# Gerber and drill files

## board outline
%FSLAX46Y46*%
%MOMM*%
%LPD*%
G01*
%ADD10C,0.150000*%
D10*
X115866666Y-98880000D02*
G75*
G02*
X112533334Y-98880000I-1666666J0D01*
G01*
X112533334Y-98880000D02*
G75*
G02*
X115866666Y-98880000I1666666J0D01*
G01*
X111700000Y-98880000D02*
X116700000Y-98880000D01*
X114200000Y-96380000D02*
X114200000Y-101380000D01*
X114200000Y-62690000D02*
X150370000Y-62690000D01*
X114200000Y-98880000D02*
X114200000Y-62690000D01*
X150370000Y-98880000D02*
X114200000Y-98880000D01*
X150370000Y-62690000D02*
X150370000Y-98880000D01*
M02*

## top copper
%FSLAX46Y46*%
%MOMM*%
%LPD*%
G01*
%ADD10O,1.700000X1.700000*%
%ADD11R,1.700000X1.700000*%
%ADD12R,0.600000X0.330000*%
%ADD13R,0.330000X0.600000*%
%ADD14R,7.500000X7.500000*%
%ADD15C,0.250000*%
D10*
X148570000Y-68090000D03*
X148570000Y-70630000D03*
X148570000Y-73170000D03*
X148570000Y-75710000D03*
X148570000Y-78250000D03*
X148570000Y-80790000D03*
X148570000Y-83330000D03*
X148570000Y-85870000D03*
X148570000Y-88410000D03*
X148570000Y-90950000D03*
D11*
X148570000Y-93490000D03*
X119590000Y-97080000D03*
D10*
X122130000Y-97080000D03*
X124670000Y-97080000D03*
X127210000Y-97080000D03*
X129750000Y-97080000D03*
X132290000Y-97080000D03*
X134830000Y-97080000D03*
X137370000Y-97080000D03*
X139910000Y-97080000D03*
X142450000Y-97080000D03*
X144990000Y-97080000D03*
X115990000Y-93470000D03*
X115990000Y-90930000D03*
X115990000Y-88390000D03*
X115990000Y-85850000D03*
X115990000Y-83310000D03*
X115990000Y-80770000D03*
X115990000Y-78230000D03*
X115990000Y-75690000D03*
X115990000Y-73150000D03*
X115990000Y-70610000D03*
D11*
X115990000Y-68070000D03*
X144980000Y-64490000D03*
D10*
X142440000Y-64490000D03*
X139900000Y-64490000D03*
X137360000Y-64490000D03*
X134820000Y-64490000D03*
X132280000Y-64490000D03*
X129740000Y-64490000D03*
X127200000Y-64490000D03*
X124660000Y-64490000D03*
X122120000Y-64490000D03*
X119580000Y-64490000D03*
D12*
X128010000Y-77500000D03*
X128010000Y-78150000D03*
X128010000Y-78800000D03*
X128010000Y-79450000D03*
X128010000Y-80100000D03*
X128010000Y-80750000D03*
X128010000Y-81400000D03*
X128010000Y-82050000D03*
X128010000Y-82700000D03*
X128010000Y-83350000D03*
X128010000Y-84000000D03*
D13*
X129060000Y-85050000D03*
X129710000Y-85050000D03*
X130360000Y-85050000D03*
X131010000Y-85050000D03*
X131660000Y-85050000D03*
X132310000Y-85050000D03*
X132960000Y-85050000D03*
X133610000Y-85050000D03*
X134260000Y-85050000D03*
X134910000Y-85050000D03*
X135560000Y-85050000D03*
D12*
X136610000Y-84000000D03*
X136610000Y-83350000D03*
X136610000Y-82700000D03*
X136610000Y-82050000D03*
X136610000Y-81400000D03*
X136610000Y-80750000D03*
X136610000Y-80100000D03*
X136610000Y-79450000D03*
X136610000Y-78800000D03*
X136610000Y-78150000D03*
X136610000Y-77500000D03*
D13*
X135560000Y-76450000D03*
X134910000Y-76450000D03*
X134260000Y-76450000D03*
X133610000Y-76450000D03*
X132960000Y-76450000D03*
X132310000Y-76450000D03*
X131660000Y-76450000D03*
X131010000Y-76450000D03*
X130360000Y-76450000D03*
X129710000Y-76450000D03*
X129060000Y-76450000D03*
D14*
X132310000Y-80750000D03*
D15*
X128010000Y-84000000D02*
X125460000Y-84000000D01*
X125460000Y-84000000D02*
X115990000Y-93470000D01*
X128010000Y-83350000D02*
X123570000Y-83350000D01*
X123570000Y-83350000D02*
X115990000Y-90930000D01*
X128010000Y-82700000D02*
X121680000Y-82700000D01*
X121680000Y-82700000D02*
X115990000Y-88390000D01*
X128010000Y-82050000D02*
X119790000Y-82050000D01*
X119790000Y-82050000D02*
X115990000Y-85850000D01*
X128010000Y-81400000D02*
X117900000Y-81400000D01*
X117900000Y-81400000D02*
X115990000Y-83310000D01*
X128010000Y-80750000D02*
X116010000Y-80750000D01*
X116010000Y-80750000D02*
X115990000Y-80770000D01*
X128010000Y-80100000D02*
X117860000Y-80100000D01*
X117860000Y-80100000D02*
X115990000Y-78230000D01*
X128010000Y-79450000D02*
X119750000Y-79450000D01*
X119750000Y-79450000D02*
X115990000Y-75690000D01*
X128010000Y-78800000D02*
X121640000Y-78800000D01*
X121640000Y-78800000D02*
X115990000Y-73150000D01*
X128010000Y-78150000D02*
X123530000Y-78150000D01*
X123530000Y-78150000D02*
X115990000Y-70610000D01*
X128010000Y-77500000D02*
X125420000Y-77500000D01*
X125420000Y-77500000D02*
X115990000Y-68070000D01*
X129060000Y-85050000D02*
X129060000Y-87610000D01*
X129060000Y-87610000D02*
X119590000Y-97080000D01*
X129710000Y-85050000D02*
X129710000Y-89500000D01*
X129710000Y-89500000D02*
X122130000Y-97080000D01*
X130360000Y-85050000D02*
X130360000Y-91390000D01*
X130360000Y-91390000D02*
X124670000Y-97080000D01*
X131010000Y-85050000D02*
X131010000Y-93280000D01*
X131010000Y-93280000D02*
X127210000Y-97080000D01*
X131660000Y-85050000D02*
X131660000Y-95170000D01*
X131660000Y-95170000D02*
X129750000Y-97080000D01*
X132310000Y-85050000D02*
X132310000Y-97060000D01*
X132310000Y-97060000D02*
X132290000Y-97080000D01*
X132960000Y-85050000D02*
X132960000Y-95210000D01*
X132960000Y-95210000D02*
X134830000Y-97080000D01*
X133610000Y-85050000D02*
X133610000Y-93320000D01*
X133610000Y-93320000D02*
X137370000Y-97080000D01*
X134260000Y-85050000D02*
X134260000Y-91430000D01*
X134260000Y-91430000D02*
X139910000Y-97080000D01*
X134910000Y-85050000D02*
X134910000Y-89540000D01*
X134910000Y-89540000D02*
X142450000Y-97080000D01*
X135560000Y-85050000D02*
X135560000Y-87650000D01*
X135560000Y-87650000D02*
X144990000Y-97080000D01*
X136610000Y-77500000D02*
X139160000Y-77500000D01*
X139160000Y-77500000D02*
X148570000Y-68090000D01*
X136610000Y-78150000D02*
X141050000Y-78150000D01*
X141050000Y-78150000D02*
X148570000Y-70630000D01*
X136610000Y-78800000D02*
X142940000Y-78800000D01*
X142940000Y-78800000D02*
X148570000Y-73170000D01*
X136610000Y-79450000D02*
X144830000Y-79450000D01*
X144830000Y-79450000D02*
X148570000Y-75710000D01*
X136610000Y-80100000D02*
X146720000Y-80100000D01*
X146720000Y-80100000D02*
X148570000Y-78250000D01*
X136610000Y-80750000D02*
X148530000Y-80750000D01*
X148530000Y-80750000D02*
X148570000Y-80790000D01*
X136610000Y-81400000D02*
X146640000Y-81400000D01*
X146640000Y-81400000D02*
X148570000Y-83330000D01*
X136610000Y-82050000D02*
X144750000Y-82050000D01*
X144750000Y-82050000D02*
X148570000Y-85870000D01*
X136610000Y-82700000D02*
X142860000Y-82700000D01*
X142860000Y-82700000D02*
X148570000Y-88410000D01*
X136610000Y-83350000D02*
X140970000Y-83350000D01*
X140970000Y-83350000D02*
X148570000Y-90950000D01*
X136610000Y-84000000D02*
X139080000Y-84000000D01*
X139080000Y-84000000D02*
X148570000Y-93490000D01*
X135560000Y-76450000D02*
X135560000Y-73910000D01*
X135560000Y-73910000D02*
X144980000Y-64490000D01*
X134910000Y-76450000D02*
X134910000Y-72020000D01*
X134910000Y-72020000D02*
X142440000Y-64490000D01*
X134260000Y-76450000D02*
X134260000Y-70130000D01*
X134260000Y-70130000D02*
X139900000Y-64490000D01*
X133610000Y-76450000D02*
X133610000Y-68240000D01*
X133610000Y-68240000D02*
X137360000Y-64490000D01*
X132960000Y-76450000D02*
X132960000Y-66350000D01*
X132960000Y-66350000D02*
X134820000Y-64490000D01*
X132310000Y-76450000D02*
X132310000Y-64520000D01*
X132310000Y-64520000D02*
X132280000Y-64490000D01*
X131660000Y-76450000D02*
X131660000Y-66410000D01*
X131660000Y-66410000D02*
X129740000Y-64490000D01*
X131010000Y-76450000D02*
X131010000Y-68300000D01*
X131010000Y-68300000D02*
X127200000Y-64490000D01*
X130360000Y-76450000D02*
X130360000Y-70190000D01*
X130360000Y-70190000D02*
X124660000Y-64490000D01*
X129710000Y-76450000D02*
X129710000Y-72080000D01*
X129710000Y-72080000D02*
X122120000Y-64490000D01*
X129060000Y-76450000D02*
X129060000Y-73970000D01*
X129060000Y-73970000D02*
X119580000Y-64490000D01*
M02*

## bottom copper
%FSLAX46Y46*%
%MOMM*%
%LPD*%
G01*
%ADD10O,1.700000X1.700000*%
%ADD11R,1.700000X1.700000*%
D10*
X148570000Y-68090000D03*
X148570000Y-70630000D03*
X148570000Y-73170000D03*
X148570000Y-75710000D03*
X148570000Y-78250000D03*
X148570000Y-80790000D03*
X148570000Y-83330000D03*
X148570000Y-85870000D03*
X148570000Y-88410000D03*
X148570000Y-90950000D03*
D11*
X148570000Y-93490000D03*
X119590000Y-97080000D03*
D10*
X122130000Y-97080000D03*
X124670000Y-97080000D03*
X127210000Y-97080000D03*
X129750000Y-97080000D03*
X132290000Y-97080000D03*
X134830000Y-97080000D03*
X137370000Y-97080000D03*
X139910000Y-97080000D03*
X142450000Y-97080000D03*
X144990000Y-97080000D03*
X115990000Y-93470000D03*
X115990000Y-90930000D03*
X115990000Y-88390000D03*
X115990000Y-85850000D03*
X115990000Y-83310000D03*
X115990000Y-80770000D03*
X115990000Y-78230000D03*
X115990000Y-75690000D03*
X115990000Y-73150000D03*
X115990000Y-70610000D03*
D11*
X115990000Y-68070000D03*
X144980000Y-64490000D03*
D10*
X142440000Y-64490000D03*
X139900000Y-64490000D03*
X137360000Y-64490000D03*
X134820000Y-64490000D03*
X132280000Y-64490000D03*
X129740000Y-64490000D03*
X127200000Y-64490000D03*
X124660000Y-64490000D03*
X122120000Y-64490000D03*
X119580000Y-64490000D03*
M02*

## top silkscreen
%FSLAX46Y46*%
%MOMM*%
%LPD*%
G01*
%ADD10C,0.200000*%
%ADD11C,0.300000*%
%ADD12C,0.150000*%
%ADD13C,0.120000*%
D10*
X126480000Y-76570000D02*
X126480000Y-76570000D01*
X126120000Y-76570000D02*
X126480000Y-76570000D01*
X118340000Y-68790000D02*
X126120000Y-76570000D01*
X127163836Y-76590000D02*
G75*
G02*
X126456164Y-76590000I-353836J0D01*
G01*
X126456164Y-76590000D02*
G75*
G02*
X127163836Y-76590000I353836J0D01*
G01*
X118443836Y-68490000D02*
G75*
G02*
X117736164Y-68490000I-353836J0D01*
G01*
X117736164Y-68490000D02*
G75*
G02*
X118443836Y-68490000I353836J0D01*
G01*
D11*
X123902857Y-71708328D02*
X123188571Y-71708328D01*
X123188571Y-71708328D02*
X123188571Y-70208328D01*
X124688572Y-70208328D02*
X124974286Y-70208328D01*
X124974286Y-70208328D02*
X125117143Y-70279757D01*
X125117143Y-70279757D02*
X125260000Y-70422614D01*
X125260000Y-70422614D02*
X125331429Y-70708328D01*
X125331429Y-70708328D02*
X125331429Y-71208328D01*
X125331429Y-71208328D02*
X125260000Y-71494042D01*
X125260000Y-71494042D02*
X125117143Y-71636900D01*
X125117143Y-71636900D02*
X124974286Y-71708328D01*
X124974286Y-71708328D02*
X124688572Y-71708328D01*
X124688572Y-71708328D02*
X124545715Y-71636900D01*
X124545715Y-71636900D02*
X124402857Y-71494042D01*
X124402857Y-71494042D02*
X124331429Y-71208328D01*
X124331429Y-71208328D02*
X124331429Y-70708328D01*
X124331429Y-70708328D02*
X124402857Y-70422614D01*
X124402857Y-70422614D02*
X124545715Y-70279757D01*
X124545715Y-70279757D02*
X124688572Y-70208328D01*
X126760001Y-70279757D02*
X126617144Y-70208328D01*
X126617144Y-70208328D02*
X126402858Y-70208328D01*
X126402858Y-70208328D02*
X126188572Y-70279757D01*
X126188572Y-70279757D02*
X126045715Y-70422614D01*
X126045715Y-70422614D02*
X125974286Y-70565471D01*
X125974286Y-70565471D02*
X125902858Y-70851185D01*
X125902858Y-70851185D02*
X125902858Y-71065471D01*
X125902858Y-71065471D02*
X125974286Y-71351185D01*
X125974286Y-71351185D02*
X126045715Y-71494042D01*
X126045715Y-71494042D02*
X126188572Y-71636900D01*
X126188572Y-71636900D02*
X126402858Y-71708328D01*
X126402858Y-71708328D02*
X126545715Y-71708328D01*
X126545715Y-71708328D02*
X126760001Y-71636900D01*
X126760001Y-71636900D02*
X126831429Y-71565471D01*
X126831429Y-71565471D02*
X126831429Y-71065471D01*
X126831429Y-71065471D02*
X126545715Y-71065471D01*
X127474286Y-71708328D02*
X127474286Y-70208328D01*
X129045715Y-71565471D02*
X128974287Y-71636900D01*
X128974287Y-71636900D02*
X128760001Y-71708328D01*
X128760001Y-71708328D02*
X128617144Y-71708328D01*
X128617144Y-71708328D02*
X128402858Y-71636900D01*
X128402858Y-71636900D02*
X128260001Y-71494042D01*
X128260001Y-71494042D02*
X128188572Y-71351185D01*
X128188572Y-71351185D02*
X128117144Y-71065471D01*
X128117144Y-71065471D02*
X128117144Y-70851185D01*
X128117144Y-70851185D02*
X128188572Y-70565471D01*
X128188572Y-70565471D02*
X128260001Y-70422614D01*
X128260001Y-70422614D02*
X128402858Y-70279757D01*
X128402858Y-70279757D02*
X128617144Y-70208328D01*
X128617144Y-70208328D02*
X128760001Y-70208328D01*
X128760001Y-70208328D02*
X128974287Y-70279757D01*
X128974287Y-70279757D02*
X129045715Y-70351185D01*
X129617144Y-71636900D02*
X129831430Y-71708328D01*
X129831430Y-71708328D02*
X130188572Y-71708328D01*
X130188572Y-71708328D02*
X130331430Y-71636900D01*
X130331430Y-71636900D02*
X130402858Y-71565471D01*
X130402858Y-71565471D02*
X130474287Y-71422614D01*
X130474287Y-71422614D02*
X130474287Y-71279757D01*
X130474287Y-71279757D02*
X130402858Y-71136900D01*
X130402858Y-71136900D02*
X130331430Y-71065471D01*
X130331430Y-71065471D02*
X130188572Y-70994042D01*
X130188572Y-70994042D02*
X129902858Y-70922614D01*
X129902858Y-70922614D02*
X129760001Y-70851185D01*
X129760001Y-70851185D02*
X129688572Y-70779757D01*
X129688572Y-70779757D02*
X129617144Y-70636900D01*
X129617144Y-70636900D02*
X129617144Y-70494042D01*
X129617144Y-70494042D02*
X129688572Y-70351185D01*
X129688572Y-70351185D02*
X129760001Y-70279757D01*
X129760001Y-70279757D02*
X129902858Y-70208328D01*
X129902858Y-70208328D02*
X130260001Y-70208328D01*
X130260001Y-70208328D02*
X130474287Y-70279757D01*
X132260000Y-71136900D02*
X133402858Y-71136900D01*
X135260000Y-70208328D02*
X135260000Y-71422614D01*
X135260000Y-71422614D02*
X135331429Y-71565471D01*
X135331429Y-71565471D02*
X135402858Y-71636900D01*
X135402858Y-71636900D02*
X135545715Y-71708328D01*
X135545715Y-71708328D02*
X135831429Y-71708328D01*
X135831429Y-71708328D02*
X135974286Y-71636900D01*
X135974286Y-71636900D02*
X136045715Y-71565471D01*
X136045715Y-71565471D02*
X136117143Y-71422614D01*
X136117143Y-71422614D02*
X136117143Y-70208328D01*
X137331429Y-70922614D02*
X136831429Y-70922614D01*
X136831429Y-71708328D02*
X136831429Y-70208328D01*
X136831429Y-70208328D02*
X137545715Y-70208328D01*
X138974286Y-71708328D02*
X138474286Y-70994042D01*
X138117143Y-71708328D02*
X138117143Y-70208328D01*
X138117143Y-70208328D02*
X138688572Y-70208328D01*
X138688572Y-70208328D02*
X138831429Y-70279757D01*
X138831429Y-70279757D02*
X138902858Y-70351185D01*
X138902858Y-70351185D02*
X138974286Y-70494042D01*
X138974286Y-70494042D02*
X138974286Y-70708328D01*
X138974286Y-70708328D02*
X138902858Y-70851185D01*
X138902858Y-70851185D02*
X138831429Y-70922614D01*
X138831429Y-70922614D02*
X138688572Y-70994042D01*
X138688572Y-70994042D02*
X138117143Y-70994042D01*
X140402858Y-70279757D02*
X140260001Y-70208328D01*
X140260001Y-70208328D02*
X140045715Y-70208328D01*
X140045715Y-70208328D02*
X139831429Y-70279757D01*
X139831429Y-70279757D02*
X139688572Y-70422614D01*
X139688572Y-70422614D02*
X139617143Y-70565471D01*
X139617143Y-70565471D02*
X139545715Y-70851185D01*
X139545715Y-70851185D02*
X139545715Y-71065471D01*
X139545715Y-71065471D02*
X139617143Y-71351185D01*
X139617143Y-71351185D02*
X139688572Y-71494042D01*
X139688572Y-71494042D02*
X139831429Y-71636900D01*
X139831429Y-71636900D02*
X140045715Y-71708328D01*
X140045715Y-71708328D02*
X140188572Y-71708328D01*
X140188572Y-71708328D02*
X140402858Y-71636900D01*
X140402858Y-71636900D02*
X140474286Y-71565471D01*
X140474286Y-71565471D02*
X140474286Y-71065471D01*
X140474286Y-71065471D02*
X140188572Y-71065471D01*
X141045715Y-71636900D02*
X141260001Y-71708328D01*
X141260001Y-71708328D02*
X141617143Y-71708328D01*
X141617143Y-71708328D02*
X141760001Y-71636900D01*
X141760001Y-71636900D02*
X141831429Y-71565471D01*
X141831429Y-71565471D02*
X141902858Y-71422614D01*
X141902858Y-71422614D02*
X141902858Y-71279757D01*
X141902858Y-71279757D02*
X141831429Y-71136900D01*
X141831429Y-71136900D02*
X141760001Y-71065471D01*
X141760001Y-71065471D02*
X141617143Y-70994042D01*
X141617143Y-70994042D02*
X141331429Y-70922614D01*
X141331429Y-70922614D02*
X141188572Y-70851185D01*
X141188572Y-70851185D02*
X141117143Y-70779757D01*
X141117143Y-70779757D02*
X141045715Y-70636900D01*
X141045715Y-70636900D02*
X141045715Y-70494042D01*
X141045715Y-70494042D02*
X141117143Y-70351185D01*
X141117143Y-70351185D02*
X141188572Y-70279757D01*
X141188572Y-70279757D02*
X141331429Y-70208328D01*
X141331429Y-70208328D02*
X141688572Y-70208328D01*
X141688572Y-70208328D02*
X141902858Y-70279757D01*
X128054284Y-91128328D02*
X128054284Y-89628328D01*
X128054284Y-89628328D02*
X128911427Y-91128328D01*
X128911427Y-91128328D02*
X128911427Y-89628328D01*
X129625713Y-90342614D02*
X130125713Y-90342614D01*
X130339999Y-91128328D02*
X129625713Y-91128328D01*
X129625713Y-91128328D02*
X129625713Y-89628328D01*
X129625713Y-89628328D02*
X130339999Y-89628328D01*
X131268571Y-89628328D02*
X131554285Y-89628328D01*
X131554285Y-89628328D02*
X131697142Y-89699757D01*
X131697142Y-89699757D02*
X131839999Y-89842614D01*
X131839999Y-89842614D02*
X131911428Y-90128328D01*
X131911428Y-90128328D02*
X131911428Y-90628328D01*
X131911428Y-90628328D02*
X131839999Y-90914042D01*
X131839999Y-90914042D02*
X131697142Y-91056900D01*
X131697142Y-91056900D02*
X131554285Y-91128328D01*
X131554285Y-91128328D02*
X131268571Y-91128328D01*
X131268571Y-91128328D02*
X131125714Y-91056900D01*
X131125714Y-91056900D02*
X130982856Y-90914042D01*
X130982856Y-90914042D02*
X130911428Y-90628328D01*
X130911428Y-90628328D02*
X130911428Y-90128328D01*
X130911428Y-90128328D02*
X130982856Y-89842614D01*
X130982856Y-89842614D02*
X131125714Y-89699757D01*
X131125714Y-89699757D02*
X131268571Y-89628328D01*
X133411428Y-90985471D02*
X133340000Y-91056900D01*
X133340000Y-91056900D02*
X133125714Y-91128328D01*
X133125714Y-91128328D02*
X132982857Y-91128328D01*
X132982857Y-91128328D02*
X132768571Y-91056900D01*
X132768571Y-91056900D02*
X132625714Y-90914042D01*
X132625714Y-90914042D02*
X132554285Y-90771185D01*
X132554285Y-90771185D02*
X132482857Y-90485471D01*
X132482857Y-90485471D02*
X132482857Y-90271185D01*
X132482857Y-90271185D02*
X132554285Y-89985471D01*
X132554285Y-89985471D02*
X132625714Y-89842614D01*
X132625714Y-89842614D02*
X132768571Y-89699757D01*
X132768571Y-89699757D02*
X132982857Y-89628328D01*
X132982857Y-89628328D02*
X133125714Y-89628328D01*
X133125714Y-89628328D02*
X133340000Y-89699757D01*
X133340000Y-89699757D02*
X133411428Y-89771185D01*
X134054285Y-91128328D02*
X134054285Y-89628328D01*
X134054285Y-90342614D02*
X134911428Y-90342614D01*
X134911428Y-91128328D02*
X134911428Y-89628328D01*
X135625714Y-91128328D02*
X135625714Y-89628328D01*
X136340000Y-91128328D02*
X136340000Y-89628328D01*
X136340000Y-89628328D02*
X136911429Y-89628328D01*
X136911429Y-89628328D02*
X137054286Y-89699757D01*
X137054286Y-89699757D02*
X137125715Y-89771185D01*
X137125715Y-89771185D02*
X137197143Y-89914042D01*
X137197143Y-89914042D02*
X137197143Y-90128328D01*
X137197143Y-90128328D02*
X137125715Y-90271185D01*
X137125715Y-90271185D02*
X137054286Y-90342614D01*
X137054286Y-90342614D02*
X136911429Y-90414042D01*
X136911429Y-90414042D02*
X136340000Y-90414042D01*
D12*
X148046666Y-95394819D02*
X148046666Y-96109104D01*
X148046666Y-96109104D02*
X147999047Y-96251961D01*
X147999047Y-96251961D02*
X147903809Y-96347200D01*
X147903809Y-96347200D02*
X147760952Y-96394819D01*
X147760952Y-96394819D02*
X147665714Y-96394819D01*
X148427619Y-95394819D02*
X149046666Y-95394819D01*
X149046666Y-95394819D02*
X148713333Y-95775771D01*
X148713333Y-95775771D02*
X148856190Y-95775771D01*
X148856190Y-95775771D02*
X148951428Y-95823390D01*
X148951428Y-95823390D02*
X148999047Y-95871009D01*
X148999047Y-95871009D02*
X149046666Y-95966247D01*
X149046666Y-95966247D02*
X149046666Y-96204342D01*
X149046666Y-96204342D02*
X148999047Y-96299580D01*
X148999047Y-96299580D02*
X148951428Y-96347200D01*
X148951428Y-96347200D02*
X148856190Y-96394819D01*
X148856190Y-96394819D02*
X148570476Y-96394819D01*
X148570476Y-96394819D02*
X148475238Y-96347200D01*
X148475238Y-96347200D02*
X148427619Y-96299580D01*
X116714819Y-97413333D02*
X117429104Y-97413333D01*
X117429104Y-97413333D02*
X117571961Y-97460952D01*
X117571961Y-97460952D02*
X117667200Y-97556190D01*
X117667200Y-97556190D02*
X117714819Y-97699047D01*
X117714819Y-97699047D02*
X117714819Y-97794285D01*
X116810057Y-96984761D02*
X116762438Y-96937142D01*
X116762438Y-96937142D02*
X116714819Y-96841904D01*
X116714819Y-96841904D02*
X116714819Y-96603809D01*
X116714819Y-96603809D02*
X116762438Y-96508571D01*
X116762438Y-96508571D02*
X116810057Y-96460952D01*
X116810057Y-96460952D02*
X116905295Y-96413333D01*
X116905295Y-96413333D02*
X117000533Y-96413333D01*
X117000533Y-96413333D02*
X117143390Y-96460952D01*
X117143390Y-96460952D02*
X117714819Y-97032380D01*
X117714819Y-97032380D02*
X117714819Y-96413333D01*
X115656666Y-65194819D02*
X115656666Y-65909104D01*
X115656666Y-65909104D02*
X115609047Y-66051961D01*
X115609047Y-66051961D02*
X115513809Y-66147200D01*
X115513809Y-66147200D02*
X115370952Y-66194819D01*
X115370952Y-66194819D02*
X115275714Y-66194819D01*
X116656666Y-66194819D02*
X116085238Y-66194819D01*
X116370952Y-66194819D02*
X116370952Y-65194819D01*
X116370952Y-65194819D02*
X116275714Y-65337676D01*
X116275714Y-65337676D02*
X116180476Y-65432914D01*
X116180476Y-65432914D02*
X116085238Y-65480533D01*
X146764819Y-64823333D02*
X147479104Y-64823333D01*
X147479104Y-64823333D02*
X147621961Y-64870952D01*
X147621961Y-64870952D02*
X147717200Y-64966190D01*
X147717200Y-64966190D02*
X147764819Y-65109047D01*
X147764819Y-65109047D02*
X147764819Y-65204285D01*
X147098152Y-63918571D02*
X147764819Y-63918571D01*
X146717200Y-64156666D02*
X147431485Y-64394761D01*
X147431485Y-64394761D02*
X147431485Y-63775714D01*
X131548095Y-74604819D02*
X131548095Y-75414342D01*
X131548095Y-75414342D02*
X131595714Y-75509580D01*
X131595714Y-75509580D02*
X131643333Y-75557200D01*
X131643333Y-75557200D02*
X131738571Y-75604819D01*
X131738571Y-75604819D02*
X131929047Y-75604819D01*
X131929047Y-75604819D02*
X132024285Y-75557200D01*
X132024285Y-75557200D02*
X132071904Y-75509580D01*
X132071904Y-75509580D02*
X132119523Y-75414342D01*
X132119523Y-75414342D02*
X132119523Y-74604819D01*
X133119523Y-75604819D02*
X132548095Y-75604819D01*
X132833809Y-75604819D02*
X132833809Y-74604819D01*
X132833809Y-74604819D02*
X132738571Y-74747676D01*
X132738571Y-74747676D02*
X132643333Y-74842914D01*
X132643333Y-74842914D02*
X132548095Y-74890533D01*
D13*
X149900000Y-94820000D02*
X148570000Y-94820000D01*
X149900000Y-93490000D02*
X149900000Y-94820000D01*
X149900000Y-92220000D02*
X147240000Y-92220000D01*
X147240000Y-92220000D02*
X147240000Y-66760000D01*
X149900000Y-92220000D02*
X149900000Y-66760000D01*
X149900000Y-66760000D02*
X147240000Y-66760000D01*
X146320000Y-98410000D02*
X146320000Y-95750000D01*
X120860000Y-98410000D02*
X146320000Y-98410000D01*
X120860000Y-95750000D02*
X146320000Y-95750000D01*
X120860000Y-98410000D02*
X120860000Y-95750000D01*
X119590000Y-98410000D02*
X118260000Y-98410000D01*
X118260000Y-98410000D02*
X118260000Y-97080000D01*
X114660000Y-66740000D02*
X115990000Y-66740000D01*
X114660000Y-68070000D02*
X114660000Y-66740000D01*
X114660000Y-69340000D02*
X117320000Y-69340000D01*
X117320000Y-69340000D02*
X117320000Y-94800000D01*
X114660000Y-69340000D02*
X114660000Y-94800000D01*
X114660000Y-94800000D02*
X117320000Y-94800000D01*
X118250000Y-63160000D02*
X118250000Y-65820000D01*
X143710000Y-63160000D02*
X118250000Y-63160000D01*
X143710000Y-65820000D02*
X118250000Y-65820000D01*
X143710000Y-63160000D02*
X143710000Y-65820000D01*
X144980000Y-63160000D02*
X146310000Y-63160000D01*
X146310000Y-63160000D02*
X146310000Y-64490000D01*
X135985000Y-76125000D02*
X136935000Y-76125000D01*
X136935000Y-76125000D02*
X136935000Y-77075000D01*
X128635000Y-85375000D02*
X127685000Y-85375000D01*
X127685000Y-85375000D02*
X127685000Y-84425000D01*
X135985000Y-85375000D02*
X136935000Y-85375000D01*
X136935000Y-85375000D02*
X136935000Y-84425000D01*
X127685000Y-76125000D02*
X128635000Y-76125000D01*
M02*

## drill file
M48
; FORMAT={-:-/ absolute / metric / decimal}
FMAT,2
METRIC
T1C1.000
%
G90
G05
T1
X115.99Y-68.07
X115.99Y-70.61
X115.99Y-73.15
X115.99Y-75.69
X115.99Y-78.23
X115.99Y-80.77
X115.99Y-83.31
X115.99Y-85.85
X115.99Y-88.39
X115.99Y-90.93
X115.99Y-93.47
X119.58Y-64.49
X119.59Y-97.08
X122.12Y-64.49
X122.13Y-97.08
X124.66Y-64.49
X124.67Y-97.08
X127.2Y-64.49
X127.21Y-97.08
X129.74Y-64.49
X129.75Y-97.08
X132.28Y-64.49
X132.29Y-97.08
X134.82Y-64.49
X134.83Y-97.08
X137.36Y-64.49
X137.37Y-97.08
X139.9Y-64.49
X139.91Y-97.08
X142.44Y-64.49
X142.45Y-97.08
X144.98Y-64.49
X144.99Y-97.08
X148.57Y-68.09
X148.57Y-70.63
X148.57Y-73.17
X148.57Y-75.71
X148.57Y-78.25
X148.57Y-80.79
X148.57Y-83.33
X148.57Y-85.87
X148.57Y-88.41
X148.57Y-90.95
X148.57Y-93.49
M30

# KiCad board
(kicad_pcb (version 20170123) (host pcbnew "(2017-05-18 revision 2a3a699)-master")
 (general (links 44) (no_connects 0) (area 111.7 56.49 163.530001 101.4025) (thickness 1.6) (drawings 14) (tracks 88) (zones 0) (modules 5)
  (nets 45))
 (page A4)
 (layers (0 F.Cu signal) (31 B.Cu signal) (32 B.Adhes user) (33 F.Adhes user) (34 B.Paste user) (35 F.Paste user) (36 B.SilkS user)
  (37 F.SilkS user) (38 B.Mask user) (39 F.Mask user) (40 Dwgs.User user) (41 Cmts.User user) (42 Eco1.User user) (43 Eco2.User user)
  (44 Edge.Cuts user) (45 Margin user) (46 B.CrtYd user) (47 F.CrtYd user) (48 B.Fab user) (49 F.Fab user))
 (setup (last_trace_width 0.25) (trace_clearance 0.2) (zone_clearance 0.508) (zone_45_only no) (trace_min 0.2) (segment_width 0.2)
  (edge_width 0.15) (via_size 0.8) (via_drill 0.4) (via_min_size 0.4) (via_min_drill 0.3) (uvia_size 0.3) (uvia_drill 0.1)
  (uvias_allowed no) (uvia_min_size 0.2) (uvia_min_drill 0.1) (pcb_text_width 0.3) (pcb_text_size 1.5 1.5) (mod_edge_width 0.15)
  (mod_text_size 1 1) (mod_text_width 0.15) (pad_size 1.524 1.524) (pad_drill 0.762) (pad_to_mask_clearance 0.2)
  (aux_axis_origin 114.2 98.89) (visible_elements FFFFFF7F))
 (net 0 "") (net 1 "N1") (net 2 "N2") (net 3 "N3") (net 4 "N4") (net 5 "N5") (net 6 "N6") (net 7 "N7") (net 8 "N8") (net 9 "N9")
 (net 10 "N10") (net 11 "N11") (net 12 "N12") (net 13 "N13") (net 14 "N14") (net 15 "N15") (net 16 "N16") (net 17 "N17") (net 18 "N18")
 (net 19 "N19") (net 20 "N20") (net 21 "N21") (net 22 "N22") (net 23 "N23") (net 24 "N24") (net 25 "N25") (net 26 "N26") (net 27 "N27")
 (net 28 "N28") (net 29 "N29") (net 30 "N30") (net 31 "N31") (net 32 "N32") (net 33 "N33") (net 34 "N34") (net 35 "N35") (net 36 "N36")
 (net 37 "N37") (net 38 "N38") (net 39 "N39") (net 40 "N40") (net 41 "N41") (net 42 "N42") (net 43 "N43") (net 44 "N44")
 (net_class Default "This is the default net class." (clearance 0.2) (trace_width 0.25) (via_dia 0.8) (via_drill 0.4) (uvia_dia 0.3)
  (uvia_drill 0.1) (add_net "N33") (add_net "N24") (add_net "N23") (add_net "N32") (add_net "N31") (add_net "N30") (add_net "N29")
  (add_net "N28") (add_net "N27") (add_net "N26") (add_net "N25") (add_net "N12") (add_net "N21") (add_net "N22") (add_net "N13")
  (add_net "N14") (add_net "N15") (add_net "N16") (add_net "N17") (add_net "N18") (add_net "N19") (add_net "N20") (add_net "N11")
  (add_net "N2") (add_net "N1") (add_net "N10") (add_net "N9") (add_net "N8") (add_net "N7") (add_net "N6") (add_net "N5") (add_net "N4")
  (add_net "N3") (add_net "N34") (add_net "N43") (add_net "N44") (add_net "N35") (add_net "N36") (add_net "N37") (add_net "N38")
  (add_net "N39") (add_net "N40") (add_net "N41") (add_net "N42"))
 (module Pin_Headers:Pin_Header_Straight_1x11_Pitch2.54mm (layer F.Cu) (at 148.57 93.49 180)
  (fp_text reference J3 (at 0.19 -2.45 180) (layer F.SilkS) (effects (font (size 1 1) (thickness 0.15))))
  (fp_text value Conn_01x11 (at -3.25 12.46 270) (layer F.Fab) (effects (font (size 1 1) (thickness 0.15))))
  (fp_line (start -1.33 -1.33) (end 0 -1.33) (layer F.SilkS) (width 0.12))
  (fp_line (start -1.33 0) (end -1.33 -1.33) (layer F.SilkS) (width 0.12))
  (fp_line (start -1.33 1.27) (end 1.33 1.27) (layer F.SilkS) (width 0.12))
  (fp_line (start 1.33 1.27) (end 1.33 26.73) (layer F.SilkS) (width 0.12))
  (fp_line (start -1.33 1.27) (end -1.33 26.73) (layer F.SilkS) (width 0.12))
  (fp_line (start -1.33 26.73) (end 1.33 26.73) (layer F.SilkS) (width 0.12))
  (pad 11 thru_hole oval (at 0 25.4 180) (size 1.7 1.7) (drill 1) (layers *.Cu *.Mask) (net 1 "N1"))
  (pad 10 thru_hole oval (at 0 22.86 180) (size 1.7 1.7) (drill 1) (layers *.Cu *.Mask) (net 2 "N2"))
  (pad 9 thru_hole oval (at 0 20.32 180) (size 1.7 1.7) (drill 1) (layers *.Cu *.Mask) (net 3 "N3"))
  (pad 8 thru_hole oval (at 0 17.78 180) (size 1.7 1.7) (drill 1) (layers *.Cu *.Mask) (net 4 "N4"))
  (pad 7 thru_hole oval (at 0 15.24 180) (size 1.7 1.7) (drill 1) (layers *.Cu *.Mask) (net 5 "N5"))
  (pad 6 thru_hole oval (at 0 12.7 180) (size 1.7 1.7) (drill 1) (layers *.Cu *.Mask) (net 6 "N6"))
  (pad 5 thru_hole oval (at 0 10.16 180) (size 1.7 1.7) (drill 1) (layers *.Cu *.Mask) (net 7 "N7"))
  (pad 4 thru_hole oval (at 0 7.62 180) (size 1.7 1.7) (drill 1) (layers *.Cu *.Mask) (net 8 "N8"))
  (pad 3 thru_hole oval (at 0 5.08 180) (size 1.7 1.7) (drill 1) (layers *.Cu *.Mask) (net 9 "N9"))
  (pad 2 thru_hole oval (at 0 2.54 180) (size 1.7 1.7) (drill 1) (layers *.Cu *.Mask) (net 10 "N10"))
  (pad 1 thru_hole rect (at 0 0 180) (size 1.7 1.7) (drill 1) (layers *.Cu *.Mask) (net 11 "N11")))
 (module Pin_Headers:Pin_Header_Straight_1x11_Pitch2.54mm (layer F.Cu) (at 119.59 97.08 90)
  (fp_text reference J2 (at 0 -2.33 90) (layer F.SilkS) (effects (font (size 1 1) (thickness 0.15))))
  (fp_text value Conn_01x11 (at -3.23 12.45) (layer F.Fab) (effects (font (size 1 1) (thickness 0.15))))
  (fp_line (start -1.33 26.73) (end 1.33 26.73) (layer F.SilkS) (width 0.12))
  (fp_line (start -1.33 1.27) (end -1.33 26.73) (layer F.SilkS) (width 0.12))
  (fp_line (start 1.33 1.27) (end 1.33 26.73) (layer F.SilkS) (width 0.12))
  (fp_line (start -1.33 1.27) (end 1.33 1.27) (layer F.SilkS) (width 0.12))
  (fp_line (start -1.33 0) (end -1.33 -1.33) (layer F.SilkS) (width 0.12))
  (fp_line (start -1.33 -1.33) (end 0 -1.33) (layer F.SilkS) (width 0.12))
  (pad 1 thru_hole rect (at 0 0 90) (size 1.7 1.7) (drill 1) (layers *.Cu *.Mask) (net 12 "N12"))
  (pad 2 thru_hole oval (at 0 2.54 90) (size 1.7 1.7) (drill 1) (layers *.Cu *.Mask) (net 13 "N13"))
  (pad 3 thru_hole oval (at 0 5.08 90) (size 1.7 1.7) (drill 1) (layers *.Cu *.Mask) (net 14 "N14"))
  (pad 4 thru_hole oval (at 0 7.62 90) (size 1.7 1.7) (drill 1) (layers *.Cu *.Mask) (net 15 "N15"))
  (pad 5 thru_hole oval (at 0 10.16 90) (size 1.7 1.7) (drill 1) (layers *.Cu *.Mask) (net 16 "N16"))
  (pad 6 thru_hole oval (at 0 12.7 90) (size 1.7 1.7) (drill 1) (layers *.Cu *.Mask) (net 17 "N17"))
  (pad 7 thru_hole oval (at 0 15.24 90) (size 1.7 1.7) (drill 1) (layers *.Cu *.Mask) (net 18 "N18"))
  (pad 8 thru_hole oval (at 0 17.78 90) (size 1.7 1.7) (drill 1) (layers *.Cu *.Mask) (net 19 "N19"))
  (pad 9 thru_hole oval (at 0 20.32 90) (size 1.7 1.7) (drill 1) (layers *.Cu *.Mask) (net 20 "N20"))
  (pad 10 thru_hole oval (at 0 22.86 90) (size 1.7 1.7) (drill 1) (layers *.Cu *.Mask) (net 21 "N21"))
  (pad 11 thru_hole oval (at 0 25.4 90) (size 1.7 1.7) (drill 1) (layers *.Cu *.Mask) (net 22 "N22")))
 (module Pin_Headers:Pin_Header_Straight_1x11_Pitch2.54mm (layer F.Cu) (at 115.99 68.07)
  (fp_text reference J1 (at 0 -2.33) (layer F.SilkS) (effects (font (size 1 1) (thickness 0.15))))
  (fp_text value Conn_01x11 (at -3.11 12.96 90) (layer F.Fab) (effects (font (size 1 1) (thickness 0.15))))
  (fp_line (start -1.33 -1.33) (end 0 -1.33) (layer F.SilkS) (width 0.12))
  (fp_line (start -1.33 0) (end -1.33 -1.33) (layer F.SilkS) (width 0.12))
  (fp_line (start -1.33 1.27) (end 1.33 1.27) (layer F.SilkS) (width 0.12))
  (fp_line (start 1.33 1.27) (end 1.33 26.73) (layer F.SilkS) (width 0.12))
  (fp_line (start -1.33 1.27) (end -1.33 26.73) (layer F.SilkS) (width 0.12))
  (fp_line (start -1.33 26.73) (end 1.33 26.73) (layer F.SilkS) (width 0.12))
  (pad 11 thru_hole oval (at 0 25.4) (size 1.7 1.7) (drill 1) (layers *.Cu *.Mask) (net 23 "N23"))
  (pad 10 thru_hole oval (at 0 22.86) (size 1.7 1.7) (drill 1) (layers *.Cu *.Mask) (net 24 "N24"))
  (pad 9 thru_hole oval (at 0 20.32) (size 1.7 1.7) (drill 1) (layers *.Cu *.Mask) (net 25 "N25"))
  (pad 8 thru_hole oval (at 0 17.78) (size 1.7 1.7) (drill 1) (layers *.Cu *.Mask) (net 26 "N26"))
  (pad 7 thru_hole oval (at 0 15.24) (size 1.7 1.7) (drill 1) (layers *.Cu *.Mask) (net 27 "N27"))
  (pad 6 thru_hole oval (at 0 12.7) (size 1.7 1.7) (drill 1) (layers *.Cu *.Mask) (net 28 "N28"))
  (pad 5 thru_hole oval (at 0 10.16) (size 1.7 1.7) (drill 1) (layers *.Cu *.Mask) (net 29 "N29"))
  (pad 4 thru_hole oval (at 0 7.62) (size 1.7 1.7) (drill 1) (layers *.Cu *.Mask) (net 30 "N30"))
  (pad 3 thru_hole oval (at 0 5.08) (size 1.7 1.7) (drill 1) (layers *.Cu *.Mask) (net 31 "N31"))
  (pad 2 thru_hole oval (at 0 2.54) (size 1.7 1.7) (drill 1) (layers *.Cu *.Mask) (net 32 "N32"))
  (pad 1 thru_hole rect (at 0 0) (size 1.7 1.7) (drill 1) (layers *.Cu *.Mask) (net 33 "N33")))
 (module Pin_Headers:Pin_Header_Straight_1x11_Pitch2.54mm (layer F.Cu) (at 144.98 64.49 270)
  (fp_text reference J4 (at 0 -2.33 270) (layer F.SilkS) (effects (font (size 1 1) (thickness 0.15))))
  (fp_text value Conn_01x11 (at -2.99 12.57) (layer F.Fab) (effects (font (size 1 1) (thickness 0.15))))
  (fp_line (start -1.33 26.73) (end 1.33 26.73) (layer F.SilkS) (width 0.12))
  (fp_line (start -1.33 1.27) (end -1.33 26.73) (layer F.SilkS) (width 0.12))
  (fp_line (start 1.33 1.27) (end 1.33 26.73) (layer F.SilkS) (width 0.12))
  (fp_line (start -1.33 1.27) (end 1.33 1.27) (layer F.SilkS) (width 0.12))
  (fp_line (start -1.33 0) (end -1.33 -1.33) (layer F.SilkS) (width 0.12))
  (fp_line (start -1.33 -1.33) (end 0 -1.33) (layer F.SilkS) (width 0.12))
  (pad 1 thru_hole rect (at 0 0 270) (size 1.7 1.7) (drill 1) (layers *.Cu *.Mask) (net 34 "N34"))
  (pad 2 thru_hole oval (at 0 2.54 270) (size 1.7 1.7) (drill 1) (layers *.Cu *.Mask) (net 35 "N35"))
  (pad 3 thru_hole oval (at 0 5.08 270) (size 1.7 1.7) (drill 1) (layers *.Cu *.Mask) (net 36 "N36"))
  (pad 4 thru_hole oval (at 0 7.62 270) (size 1.7 1.7) (drill 1) (layers *.Cu *.Mask) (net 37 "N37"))
  (pad 5 thru_hole oval (at 0 10.16 270) (size 1.7 1.7) (drill 1) (layers *.Cu *.Mask) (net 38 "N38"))
  (pad 6 thru_hole oval (at 0 12.7 270) (size 1.7 1.7) (drill 1) (layers *.Cu *.Mask) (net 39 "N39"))
  (pad 7 thru_hole oval (at 0 15.24 270) (size 1.7 1.7) (drill 1) (layers *.Cu *.Mask) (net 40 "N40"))
  (pad 8 thru_hole oval (at 0 17.78 270) (size 1.7 1.7) (drill 1) (layers *.Cu *.Mask) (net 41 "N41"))
  (pad 9 thru_hole oval (at 0 20.32 270) (size 1.7 1.7) (drill 1) (layers *.Cu *.Mask) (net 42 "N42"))
  (pad 10 thru_hole oval (at 0 22.86 270) (size 1.7 1.7) (drill 1) (layers *.Cu *.Mask) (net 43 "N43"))
  (pad 11 thru_hole oval (at 0 25.4 270) (size 1.7 1.7) (drill 1) (layers *.Cu *.Mask) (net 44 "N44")))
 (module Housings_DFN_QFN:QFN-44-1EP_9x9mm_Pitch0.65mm (layer F.Cu) (at 132.31 80.75)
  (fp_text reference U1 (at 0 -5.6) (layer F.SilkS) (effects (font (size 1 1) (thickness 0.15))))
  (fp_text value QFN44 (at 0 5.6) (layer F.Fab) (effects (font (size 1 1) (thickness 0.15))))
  (fp_line (start 3.675 -4.625) (end 4.625 -4.625) (layer F.SilkS) (width 0.12))
  (fp_line (start 4.625 -4.625) (end 4.625 -3.675) (layer F.SilkS) (width 0.12))
  (fp_line (start -3.675 4.625) (end -4.625 4.625) (layer F.SilkS) (width 0.12))
  (fp_line (start -4.625 4.625) (end -4.625 3.675) (layer F.SilkS) (width 0.12))
  (fp_line (start 3.675 4.625) (end 4.625 4.625) (layer F.SilkS) (width 0.12))
  (fp_line (start 4.625 4.625) (end 4.625 3.675) (layer F.SilkS) (width 0.12))
  (fp_line (start -4.625 -4.625) (end -3.675 -4.625) (layer F.SilkS) (width 0.12))
  (pad 1 smd rect (at -4.3 -3.25) (size 0.6 0.33) (layers F.Cu F.Paste F.Mask) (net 33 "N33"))
  (pad 2 smd rect (at -4.3 -2.6) (size 0.6 0.33) (layers F.Cu F.Paste F.Mask) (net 32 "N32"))
  (pad 3 smd rect (at -4.3 -1.95) (size 0.6 0.33) (layers F.Cu F.Paste F.Mask) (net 31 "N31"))
  (pad 4 smd rect (at -4.3 -1.3) (size 0.6 0.33) (layers F.Cu F.Paste F.Mask) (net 30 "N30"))
  (pad 5 smd rect (at -4.3 -0.65) (size 0.6 0.33) (layers F.Cu F.Paste F.Mask) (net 29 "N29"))
  (pad 6 smd rect (at -4.3 0) (size 0.6 0.33) (layers F.Cu F.Paste F.Mask) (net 28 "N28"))
  (pad 7 smd rect (at -4.3 0.65) (size 0.6 0.33) (layers F.Cu F.Paste F.Mask) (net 27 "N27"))
  (pad 8 smd rect (at -4.3 1.3) (size 0.6 0.33) (layers F.Cu F.Paste F.Mask) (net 26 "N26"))
  (pad 9 smd rect (at -4.3 1.95) (size 0.6 0.33) (layers F.Cu F.Paste F.Mask) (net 25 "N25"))
  (pad 10 smd rect (at -4.3 2.6) (size 0.6 0.33) (layers F.Cu F.Paste F.Mask) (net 24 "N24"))
  (pad 11 smd rect (at -4.3 3.25) (size 0.6 0.33) (layers F.Cu F.Paste F.Mask) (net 23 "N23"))
  (pad 12 smd rect (at -3.25 4.3 90) (size 0.6 0.33) (layers F.Cu F.Paste F.Mask) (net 12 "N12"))
  (pad 13 smd rect (at -2.6 4.3 90) (size 0.6 0.33) (layers F.Cu F.Paste F.Mask) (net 13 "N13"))
  (pad 14 smd rect (at -1.95 4.3 90) (size 0.6 0.33) (layers F.Cu F.Paste F.Mask) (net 14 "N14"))
  (pad 15 smd rect (at -1.3 4.3 90) (size 0.6 0.33) (layers F.Cu F.Paste F.Mask) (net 15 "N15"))
  (pad 16 smd rect (at -0.65 4.3 90) (size 0.6 0.33) (layers F.Cu F.Paste F.Mask) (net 16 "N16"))
  (pad 17 smd rect (at 0 4.3 90) (size 0.6 0.33) (layers F.Cu F.Paste F.Mask) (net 17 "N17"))
  (pad 18 smd rect (at 0.65 4.3 90) (size 0.6 0.33) (layers F.Cu F.Paste F.Mask) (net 18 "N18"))
  (pad 19 smd rect (at 1.3 4.3 90) (size 0.6 0.33) (layers F.Cu F.Paste F.Mask) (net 19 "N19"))
  (pad 20 smd rect (at 1.95 4.3 90) (size 0.6 0.33) (layers F.Cu F.Paste F.Mask) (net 20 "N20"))
  (pad 21 smd rect (at 2.6 4.3 90) (size 0.6 0.33) (layers F.Cu F.Paste F.Mask) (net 21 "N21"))
  (pad 22 smd rect (at 3.25 4.3 90) (size 0.6 0.33) (layers F.Cu F.Paste F.Mask) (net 22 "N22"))
  (pad 23 smd rect (at 4.3 3.25) (size 0.6 0.33) (layers F.Cu F.Paste F.Mask) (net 11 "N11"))
  (pad 24 smd rect (at 4.3 2.6) (size 0.6 0.33) (layers F.Cu F.Paste F.Mask) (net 10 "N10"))
  (pad 25 smd rect (at 4.3 1.95) (size 0.6 0.33) (layers F.Cu F.Paste F.Mask) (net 9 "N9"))
  (pad 26 smd rect (at 4.3 1.3) (size 0.6 0.33) (layers F.Cu F.Paste F.Mask) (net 8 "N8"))
  (pad 27 smd rect (at 4.3 0.65) (size 0.6 0.33) (layers F.Cu F.Paste F.Mask) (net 7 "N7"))
  (pad 28 smd rect (at 4.3 0) (size 0.6 0.33) (layers F.Cu F.Paste F.Mask) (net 6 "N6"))
  (pad 29 smd rect (at 4.3 -0.65) (size 0.6 0.33) (layers F.Cu F.Paste F.Mask) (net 5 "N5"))
  (pad 30 smd rect (at 4.3 -1.3) (size 0.6 0.33) (layers F.Cu F.Paste F.Mask) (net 4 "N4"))
  (pad 31 smd rect (at 4.3 -1.95) (size 0.6 0.33) (layers F.Cu F.Paste F.Mask) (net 3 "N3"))
  (pad 32 smd rect (at 4.3 -2.6) (size 0.6 0.33) (layers F.Cu F.Paste F.Mask) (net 2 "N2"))
  (pad 33 smd rect (at 4.3 -3.25) (size 0.6 0.33) (layers F.Cu F.Paste F.Mask) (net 1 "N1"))
  (pad 34 smd rect (at 3.25 -4.3 90) (size 0.6 0.33) (layers F.Cu F.Paste F.Mask) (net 34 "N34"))
  (pad 35 smd rect (at 2.6 -4.3 90) (size 0.6 0.33) (layers F.Cu F.Paste F.Mask) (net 35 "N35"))
  (pad 36 smd rect (at 1.95 -4.3 90) (size 0.6 0.33) (layers F.Cu F.Paste F.Mask) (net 36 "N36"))
  (pad 37 smd rect (at 1.3 -4.3 90) (size 0.6 0.33) (layers F.Cu F.Paste F.Mask) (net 37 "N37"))
  (pad 38 smd rect (at 0.65 -4.3 90) (size 0.6 0.33) (layers F.Cu F.Paste F.Mask) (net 38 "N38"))
  (pad 39 smd rect (at 0 -4.3 90) (size 0.6 0.33) (layers F.Cu F.Paste F.Mask) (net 39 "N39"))
  (pad 40 smd rect (at -0.65 -4.3 90) (size 0.6 0.33) (layers F.Cu F.Paste F.Mask) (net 40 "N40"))
  (pad 41 smd rect (at -1.3 -4.3 90) (size 0.6 0.33) (layers F.Cu F.Paste F.Mask) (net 41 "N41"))
  (pad 42 smd rect (at -1.95 -4.3 90) (size 0.6 0.33) (layers F.Cu F.Paste F.Mask) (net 42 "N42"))
  (pad 43 smd rect (at -2.6 -4.3 90) (size 0.6 0.33) (layers F.Cu F.Paste F.Mask) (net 43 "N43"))
  (pad 44 smd rect (at -3.25 -4.3 90) (size 0.6 0.33) (layers F.Cu F.Paste F.Mask) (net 44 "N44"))
  (pad 45 smd rect (at 0 0) (size 7.5 7.5) (layers F.Cu F.Mask))
  (pad "" smd rect (at -1.875 -1.875) (size 2.65 2.65) (layers F.Paste))
  (pad "" smd rect (at -1.875 1.875) (size 2.65 2.65) (layers F.Paste))
  (pad "" smd rect (at 1.875 -1.875) (size 2.65 2.65) (layers F.Paste))
  (pad "" smd rect (at 1.875 1.875) (size 2.65 2.65) (layers F.Paste)))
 (gr_line (start 126.48 76.57) (end 126.48 76.57) (layer F.SilkS) (width 0.2))
 (gr_line (start 126.12 76.57) (end 126.48 76.57) (layer F.SilkS) (width 0.2))
 (gr_line (start 118.34 68.79) (end 126.12 76.57) (layer F.SilkS) (width 0.2))
 (gr_circle (center 126.81 76.59) (end 126.55 76.35) (layer F.SilkS) (width 0.2))
 (gr_circle (center 118.09 68.49) (end 117.83 68.25) (layer F.SilkS) (width 0.2))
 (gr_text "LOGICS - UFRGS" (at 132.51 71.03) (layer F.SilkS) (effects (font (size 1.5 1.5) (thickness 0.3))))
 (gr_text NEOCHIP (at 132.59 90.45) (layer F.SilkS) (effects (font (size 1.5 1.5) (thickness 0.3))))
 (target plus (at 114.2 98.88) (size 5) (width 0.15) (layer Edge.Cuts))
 (gr_line (start 114.2 62.69) (end 150.37 62.69) (layer Edge.Cuts) (width 0.15))
 (gr_line (start 114.2 98.88) (end 114.2 62.69) (layer Edge.Cuts) (width 0.15))
 (gr_line (start 150.37 98.88) (end 114.2 98.88) (layer Edge.Cuts) (width 0.15))
 (gr_line (start 150.37 62.69) (end 150.37 98.88) (layer Edge.Cuts) (width 0.15))
 (segment (start 128.01 84) (end 125.46 84) (width 0.25) (layer F.Cu) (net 23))
 (segment (start 125.46 84) (end 115.99 93.47) (width 0.25) (layer F.Cu) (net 23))
 (segment (start 128.01 83.35) (end 123.57 83.35) (width 0.25) (layer F.Cu) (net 24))
 (segment (start 123.57 83.35) (end 115.99 90.93) (width 0.25) (layer F.Cu) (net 24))
 (segment (start 128.01 82.7) (end 121.68 82.7) (width 0.25) (layer F.Cu) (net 25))
 (segment (start 121.68 82.7) (end 115.99 88.39) (width 0.25) (layer F.Cu) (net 25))
 (segment (start 128.01 82.05) (end 119.79 82.05) (width 0.25) (layer F.Cu) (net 26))
 (segment (start 119.79 82.05) (end 115.99 85.85) (width 0.25) (layer F.Cu) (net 26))
 (segment (start 128.01 81.4) (end 117.9 81.4) (width 0.25) (layer F.Cu) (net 27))
 (segment (start 117.9 81.4) (end 115.99 83.31) (width 0.25) (layer F.Cu) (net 27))
 (segment (start 128.01 80.75) (end 116.01 80.75) (width 0.25) (layer F.Cu) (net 28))
 (segment (start 116.01 80.75) (end 115.99 80.77) (width 0.25) (layer F.Cu) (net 28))
 (segment (start 128.01 80.1) (end 117.86 80.1) (width 0.25) (layer F.Cu) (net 29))
 (segment (start 117.86 80.1) (end 115.99 78.23) (width 0.25) (layer F.Cu) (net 29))
 (segment (start 128.01 79.45) (end 119.75 79.45) (width 0.25) (layer F.Cu) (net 30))
 (segment (start 119.75 79.45) (end 115.99 75.69) (width 0.25) (layer F.Cu) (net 30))
 (segment (start 128.01 78.8) (end 121.64 78.8) (width 0.25) (layer F.Cu) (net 31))
 (segment (start 121.64 78.8) (end 115.99 73.15) (width 0.25) (layer F.Cu) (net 31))
 (segment (start 128.01 78.15) (end 123.53 78.15) (width 0.25) (layer F.Cu) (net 32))
 (segment (start 123.53 78.15) (end 115.99 70.61) (width 0.25) (layer F.Cu) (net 32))
 (segment (start 128.01 77.5) (end 125.42 77.5) (width 0.25) (layer F.Cu) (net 33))
 (segment (start 125.42 77.5) (end 115.99 68.07) (width 0.25) (layer F.Cu) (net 33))
 (segment (start 129.06 85.05) (end 129.06 87.61) (width 0.25) (layer F.Cu) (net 12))
 (segment (start 129.06 87.61) (end 119.59 97.08) (width 0.25) (layer F.Cu) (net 12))
 (segment (start 129.71 85.05) (end 129.71 89.5) (width 0.25) (layer F.Cu) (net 13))
 (segment (start 129.71 89.5) (end 122.13 97.08) (width 0.25) (layer F.Cu) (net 13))
 (segment (start 130.36 85.05) (end 130.36 91.39) (width 0.25) (layer F.Cu) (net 14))
 (segment (start 130.36 91.39) (end 124.67 97.08) (width 0.25) (layer F.Cu) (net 14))
 (segment (start 131.01 85.05) (end 131.01 93.28) (width 0.25) (layer F.Cu) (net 15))
 (segment (start 131.01 93.28) (end 127.21 97.08) (width 0.25) (layer F.Cu) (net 15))
 (segment (start 131.66 85.05) (end 131.66 95.17) (width 0.25) (layer F.Cu) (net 16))
 (segment (start 131.66 95.17) (end 129.75 97.08) (width 0.25) (layer F.Cu) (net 16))
 (segment (start 132.31 85.05) (end 132.31 97.06) (width 0.25) (layer F.Cu) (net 17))
 (segment (start 132.31 97.06) (end 132.29 97.08) (width 0.25) (layer F.Cu) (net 17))
 (segment (start 132.96 85.05) (end 132.96 95.21) (width 0.25) (layer F.Cu) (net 18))
 (segment (start 132.96 95.21) (end 134.83 97.08) (width 0.25) (layer F.Cu) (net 18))
 (segment (start 133.61 85.05) (end 133.61 93.32) (width 0.25) (layer F.Cu) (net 19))
 (segment (start 133.61 93.32) (end 137.37 97.08) (width 0.25) (layer F.Cu) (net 19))
 (segment (start 134.26 85.05) (end 134.26 91.43) (width 0.25) (layer F.Cu) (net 20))
 (segment (start 134.26 91.43) (end 139.91 97.08) (width 0.25) (layer F.Cu) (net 20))
 (segment (start 134.91 85.05) (end 134.91 89.54) (width 0.25) (layer F.Cu) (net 21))
 (segment (start 134.91 89.54) (end 142.45 97.08) (width 0.25) (layer F.Cu) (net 21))
 (segment (start 135.56 85.05) (end 135.56 87.65) (width 0.25) (layer F.Cu) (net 22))
 (segment (start 135.56 87.65) (end 144.99 97.08) (width 0.25) (layer F.Cu) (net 22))
 (segment (start 136.61 77.5) (end 139.16 77.5) (width 0.25) (layer F.Cu) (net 1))
 (segment (start 139.16 77.5) (end 148.57 68.09) (width 0.25) (layer F.Cu) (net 1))
 (segment (start 136.61 78.15) (end 141.05 78.15) (width 0.25) (layer F.Cu) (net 2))
 (segment (start 141.05 78.15) (end 148.57 70.63) (width 0.25) (layer F.Cu) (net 2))
 (segment (start 136.61 78.8) (end 142.94 78.8) (width 0.25) (layer F.Cu) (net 3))
 (segment (start 142.94 78.8) (end 148.57 73.17) (width 0.25) (layer F.Cu) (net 3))
 (segment (start 136.61 79.45) (end 144.83 79.45) (width 0.25) (layer F.Cu) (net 4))
 (segment (start 144.83 79.45) (end 148.57 75.71) (width 0.25) (layer F.Cu) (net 4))
 (segment (start 136.61 80.1) (end 146.72 80.1) (width 0.25) (layer F.Cu) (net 5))
 (segment (start 146.72 80.1) (end 148.57 78.25) (width 0.25) (layer F.Cu) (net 5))
 (segment (start 136.61 80.75) (end 148.53 80.75) (width 0.25) (layer F.Cu) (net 6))
 (segment (start 148.53 80.75) (end 148.57 80.79) (width 0.25) (layer F.Cu) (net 6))
 (segment (start 136.61 81.4) (end 146.64 81.4) (width 0.25) (layer F.Cu) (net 7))
 (segment (start 146.64 81.4) (end 148.57 83.33) (width 0.25) (layer F.Cu) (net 7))
 (segment (start 136.61 82.05) (end 144.75 82.05) (width 0.25) (layer F.Cu) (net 8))
 (segment (start 144.75 82.05) (end 148.57 85.87) (width 0.25) (layer F.Cu) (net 8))
 (segment (start 136.61 82.7) (end 142.86 82.7) (width 0.25) (layer F.Cu) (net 9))
 (segment (start 142.86 82.7) (end 148.57 88.41) (width 0.25) (layer F.Cu) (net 9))
 (segment (start 136.61 83.35) (end 140.97 83.35) (width 0.25) (layer F.Cu) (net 10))
 (segment (start 140.97 83.35) (end 148.57 90.95) (width 0.25) (layer F.Cu) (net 10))
 (segment (start 136.61 84) (end 139.08 84) (width 0.25) (layer F.Cu) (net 11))
 (segment (start 139.08 84) (end 148.57 93.49) (width 0.25) (layer F.Cu) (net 11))
 (segment (start 135.56 76.45) (end 135.56 73.91) (width 0.25) (layer F.Cu) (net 34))
 (segment (start 135.56 73.91) (end 144.98 64.49) (width 0.25) (layer F.Cu) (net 34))
 (segment (start 134.91 76.45) (end 134.91 72.02) (width 0.25) (layer F.Cu) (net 35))
 (segment (start 134.91 72.02) (end 142.44 64.49) (width 0.25) (layer F.Cu) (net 35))
 (segment (start 134.26 76.45) (end 134.26 70.13) (width 0.25) (layer F.Cu) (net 36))
 (segment (start 134.26 70.13) (end 139.9 64.49) (width 0.25) (layer F.Cu) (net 36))
 (segment (start 133.61 76.45) (end 133.61 68.24) (width 0.25) (layer F.Cu) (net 37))
 (segment (start 133.61 68.24) (end 137.36 64.49) (width 0.25) (layer F.Cu) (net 37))
 (segment (start 132.96 76.45) (end 132.96 66.35) (width 0.25) (layer F.Cu) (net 38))
 (segment (start 132.96 66.35) (end 134.82 64.49) (width 0.25) (layer F.Cu) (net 38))
 (segment (start 132.31 76.45) (end 132.31 64.52) (width 0.25) (layer F.Cu) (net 39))
 (segment (start 132.31 64.52) (end 132.28 64.49) (width 0.25) (layer F.Cu) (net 39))
 (segment (start 131.66 76.45) (end 131.66 66.41) (width 0.25) (layer F.Cu) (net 40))
 (segment (start 131.66 66.41) (end 129.74 64.49) (width 0.25) (layer F.Cu) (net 40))
 (segment (start 131.01 76.45) (end 131.01 68.3) (width 0.25) (layer F.Cu) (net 41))
 (segment (start 131.01 68.3) (end 127.2 64.49) (width 0.25) (layer F.Cu) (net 41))
 (segment (start 130.36 76.45) (end 130.36 70.19) (width 0.25) (layer F.Cu) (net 42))
 (segment (start 130.36 70.19) (end 124.66 64.49) (width 0.25) (layer F.Cu) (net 42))
 (segment (start 129.71 76.45) (end 129.71 72.08) (width 0.25) (layer F.Cu) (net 43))
 (segment (start 129.71 72.08) (end 122.12 64.49) (width 0.25) (layer F.Cu) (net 43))
 (segment (start 129.06 76.45) (end 129.06 73.97) (width 0.25) (layer F.Cu) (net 44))
 (segment (start 129.06 73.97) (end 119.58 64.49) (width 0.25) (layer F.Cu) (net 44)))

